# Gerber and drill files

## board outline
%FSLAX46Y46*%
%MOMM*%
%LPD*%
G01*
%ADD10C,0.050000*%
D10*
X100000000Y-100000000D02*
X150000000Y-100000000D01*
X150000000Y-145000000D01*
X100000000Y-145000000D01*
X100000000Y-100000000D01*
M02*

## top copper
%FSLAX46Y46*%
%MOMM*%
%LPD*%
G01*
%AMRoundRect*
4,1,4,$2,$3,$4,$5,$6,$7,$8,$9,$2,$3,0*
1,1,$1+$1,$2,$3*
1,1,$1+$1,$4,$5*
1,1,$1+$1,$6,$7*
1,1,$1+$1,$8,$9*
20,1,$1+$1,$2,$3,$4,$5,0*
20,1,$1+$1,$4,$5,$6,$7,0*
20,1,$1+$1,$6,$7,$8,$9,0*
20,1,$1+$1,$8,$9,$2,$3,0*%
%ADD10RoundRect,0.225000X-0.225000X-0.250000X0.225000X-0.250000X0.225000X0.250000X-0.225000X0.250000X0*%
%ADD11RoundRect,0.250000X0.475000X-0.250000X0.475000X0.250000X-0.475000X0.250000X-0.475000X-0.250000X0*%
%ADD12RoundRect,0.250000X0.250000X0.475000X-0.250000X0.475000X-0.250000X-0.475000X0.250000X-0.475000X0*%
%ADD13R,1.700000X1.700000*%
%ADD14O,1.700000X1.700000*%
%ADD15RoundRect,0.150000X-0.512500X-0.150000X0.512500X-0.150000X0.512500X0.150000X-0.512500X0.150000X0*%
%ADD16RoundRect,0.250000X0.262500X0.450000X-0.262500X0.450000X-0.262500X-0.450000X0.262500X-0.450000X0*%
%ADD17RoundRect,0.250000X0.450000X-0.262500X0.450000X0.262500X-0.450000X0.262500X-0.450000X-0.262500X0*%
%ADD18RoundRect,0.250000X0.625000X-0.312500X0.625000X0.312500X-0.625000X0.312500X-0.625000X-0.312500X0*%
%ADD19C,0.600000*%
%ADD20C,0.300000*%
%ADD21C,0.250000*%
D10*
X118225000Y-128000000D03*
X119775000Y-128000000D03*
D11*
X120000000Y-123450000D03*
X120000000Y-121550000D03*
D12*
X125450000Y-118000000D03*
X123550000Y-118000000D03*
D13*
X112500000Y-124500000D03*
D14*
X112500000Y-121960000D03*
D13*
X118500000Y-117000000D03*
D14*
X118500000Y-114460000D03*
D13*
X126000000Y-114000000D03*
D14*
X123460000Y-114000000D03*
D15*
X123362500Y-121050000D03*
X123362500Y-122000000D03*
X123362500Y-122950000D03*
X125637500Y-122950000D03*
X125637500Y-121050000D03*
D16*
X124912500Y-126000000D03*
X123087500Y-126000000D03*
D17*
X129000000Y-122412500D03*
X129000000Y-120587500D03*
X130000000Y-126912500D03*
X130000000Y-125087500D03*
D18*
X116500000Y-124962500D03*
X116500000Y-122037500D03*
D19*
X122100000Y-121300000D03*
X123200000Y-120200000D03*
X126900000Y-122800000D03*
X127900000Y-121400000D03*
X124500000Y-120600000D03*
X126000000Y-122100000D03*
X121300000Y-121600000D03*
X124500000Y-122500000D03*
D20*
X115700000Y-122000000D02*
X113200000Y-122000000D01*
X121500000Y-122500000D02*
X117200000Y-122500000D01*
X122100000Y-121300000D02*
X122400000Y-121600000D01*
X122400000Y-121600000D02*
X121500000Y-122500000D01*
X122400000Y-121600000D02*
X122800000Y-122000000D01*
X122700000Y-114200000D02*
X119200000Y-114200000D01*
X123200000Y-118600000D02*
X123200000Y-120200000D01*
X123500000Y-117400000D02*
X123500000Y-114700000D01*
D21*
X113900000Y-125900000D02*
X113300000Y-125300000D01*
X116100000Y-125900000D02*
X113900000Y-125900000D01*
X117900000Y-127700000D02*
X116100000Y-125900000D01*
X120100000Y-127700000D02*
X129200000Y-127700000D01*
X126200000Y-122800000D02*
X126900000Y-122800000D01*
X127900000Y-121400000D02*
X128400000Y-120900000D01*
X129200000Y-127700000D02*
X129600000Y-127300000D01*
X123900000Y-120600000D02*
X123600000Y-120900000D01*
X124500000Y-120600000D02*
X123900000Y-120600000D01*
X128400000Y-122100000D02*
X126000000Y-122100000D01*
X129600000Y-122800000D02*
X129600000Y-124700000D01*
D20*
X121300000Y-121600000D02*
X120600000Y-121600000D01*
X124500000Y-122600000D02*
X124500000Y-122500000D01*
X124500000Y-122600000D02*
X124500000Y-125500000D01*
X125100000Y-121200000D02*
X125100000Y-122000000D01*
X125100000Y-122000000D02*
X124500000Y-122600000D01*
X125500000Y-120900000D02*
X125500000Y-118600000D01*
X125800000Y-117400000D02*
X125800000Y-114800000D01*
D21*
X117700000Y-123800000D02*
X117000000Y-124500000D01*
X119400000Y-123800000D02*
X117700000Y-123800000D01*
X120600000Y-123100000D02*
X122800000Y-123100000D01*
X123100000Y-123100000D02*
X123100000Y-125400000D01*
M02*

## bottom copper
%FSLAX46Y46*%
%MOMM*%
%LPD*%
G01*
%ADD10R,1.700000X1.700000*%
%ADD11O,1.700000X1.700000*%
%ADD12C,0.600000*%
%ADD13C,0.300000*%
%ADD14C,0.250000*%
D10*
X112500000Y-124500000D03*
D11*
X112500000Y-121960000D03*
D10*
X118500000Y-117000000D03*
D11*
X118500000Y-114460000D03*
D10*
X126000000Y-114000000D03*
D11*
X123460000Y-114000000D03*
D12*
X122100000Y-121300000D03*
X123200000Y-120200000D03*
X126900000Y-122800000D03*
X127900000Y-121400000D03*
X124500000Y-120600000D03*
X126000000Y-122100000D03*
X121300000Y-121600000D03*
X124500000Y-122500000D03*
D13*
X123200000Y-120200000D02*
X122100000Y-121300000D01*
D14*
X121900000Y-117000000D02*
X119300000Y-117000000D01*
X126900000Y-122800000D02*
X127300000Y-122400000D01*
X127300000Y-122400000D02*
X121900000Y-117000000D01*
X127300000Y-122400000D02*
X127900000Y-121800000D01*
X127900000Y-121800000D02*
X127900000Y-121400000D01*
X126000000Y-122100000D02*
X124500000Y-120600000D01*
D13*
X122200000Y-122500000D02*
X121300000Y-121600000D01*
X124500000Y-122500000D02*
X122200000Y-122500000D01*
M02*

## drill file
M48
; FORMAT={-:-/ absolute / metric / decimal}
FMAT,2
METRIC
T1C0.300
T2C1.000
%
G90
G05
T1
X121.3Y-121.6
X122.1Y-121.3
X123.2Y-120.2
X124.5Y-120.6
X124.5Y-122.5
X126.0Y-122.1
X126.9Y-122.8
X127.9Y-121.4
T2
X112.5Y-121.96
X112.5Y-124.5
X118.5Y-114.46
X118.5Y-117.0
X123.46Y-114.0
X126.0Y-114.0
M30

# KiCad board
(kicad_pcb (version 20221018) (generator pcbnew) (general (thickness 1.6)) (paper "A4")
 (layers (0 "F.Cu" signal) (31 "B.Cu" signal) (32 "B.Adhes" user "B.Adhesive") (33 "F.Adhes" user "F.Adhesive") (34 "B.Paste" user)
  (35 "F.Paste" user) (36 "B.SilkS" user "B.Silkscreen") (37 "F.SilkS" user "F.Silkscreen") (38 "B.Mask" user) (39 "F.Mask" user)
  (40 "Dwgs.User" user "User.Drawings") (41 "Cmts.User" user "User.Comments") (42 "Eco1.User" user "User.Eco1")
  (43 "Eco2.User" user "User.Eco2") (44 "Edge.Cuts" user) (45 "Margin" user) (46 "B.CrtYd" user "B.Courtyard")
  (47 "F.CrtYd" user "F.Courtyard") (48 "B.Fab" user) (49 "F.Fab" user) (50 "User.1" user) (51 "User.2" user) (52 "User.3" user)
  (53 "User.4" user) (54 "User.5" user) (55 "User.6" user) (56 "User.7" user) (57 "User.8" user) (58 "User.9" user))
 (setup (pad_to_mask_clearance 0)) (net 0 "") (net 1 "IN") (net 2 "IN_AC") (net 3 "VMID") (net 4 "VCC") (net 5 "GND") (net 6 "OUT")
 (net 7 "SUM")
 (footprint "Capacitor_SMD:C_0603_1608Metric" (layer "F.Cu") (at 119 128)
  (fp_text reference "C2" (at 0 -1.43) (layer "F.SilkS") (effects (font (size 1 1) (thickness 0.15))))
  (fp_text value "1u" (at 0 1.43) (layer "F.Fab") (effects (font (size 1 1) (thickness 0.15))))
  (pad "1" smd roundrect (at -0.775 0) (size 0.9 0.95) (layers "F.Cu" "F.Paste" "F.Mask") (roundrect_rratio 0.25) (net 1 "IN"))
  (pad "2" smd roundrect (at 0.775 0) (size 0.9 0.95) (layers "F.Cu" "F.Paste" "F.Mask") (roundrect_rratio 0.25) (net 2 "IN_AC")))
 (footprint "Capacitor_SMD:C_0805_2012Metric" (layer "F.Cu") (at 120 122.5 90)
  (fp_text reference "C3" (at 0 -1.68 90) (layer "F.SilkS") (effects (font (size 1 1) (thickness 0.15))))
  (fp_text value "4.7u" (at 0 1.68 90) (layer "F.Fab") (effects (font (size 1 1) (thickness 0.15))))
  (pad "1" smd roundrect (at -0.95 0 90) (size 1 1.45) (layers "F.Cu" "F.Paste" "F.Mask") (roundrect_rratio 0.25) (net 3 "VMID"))
  (pad "2" smd roundrect (at 0.95 0 90) (size 1 1.45) (layers "F.Cu" "F.Paste" "F.Mask") (roundrect_rratio 0.25) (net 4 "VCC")))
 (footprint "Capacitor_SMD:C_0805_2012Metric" (layer "F.Cu") (at 124.5 118 180)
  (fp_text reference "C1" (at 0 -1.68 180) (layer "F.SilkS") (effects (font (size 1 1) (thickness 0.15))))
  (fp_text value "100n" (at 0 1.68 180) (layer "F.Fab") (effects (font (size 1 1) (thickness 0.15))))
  (pad "1" smd roundrect (at -0.95 0 180) (size 1 1.45) (layers "F.Cu" "F.Paste" "F.Mask") (roundrect_rratio 0.25) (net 4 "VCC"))
  (pad "2" smd roundrect (at 0.95 0 180) (size 1 1.45) (layers "F.Cu" "F.Paste" "F.Mask") (roundrect_rratio 0.25) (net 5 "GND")))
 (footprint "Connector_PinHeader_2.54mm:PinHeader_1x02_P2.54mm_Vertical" (layer "F.Cu") (at 112.5 124.5 180)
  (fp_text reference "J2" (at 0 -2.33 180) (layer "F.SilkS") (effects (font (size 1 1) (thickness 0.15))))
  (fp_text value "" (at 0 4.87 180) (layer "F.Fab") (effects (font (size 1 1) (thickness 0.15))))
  (pad "1" thru_hole rect (at 0 0 180) (size 1.7 1.7) (drill 1) (layers "*.Cu" "*.Mask") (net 1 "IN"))
  (pad "2" thru_hole oval (at 0 2.54 180) (size 1.7 1.7) (drill 1) (layers "*.Cu" "*.Mask") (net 5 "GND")))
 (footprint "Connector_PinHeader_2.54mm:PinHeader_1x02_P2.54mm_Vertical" (layer "F.Cu") (at 118.5 117 180)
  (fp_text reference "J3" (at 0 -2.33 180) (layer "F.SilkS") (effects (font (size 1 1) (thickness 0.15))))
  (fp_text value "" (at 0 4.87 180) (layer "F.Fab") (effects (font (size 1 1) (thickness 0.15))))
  (pad "1" thru_hole rect (at 0 0 180) (size 1.7 1.7) (drill 1) (layers "*.Cu" "*.Mask") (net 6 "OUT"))
  (pad "2" thru_hole oval (at 0 2.54 180) (size 1.7 1.7) (drill 1) (layers "*.Cu" "*.Mask") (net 5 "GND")))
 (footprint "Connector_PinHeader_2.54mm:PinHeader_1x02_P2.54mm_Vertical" (layer "F.Cu") (at 126 114 -90)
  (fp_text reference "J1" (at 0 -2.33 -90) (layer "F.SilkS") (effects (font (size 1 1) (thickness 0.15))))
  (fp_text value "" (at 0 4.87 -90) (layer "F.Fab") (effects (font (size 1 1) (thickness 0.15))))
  (pad "1" thru_hole rect (at 0 0 270) (size 1.7 1.7) (drill 1) (layers "*.Cu" "*.Mask") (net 4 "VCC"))
  (pad "2" thru_hole oval (at 0 2.54 270) (size 1.7 1.7) (drill 1) (layers "*.Cu" "*.Mask") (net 5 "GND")))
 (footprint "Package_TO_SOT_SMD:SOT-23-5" (layer "F.Cu") (at 124.5 122)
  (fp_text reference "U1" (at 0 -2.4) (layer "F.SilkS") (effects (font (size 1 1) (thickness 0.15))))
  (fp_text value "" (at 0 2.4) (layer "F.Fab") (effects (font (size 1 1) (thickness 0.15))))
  (pad "1" smd roundrect (at -1.1375 -0.95) (size 1.325 0.6) (layers "F.Cu" "F.Paste" "F.Mask") (roundrect_rratio 0.25) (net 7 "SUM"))
  (pad "2" smd roundrect (at -1.1375 0) (size 1.325 0.6) (layers "F.Cu" "F.Paste" "F.Mask") (roundrect_rratio 0.25) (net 5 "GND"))
  (pad "3" smd roundrect (at -1.1375 0.95) (size 1.325 0.6) (layers "F.Cu" "F.Paste" "F.Mask") (roundrect_rratio 0.25) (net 3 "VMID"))
  (pad "4" smd roundrect (at 1.1375 0.95) (size 1.325 0.6) (layers "F.Cu" "F.Paste" "F.Mask") (roundrect_rratio 0.25) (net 6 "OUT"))
  (pad "5" smd roundrect (at 1.1375 -0.95) (size 1.325 0.6) (layers "F.Cu" "F.Paste" "F.Mask") (roundrect_rratio 0.25) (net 4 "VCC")))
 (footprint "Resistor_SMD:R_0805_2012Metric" (layer "F.Cu") (at 124 126 180)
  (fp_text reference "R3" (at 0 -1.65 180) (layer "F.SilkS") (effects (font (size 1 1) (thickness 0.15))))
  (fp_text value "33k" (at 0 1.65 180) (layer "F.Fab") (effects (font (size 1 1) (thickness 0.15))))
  (pad "1" smd roundrect (at -0.9125 0 180) (size 1.025 1.4) (layers "F.Cu" "F.Paste" "F.Mask") (roundrect_rratio 0.243902) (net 4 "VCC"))
  (pad "2" smd roundrect (at 0.9125 0 180) (size 1.025 1.4) (layers "F.Cu" "F.Paste" "F.Mask") (roundrect_rratio 0.243902) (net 3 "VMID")))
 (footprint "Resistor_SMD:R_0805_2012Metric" (layer "F.Cu") (at 129 121.5 90)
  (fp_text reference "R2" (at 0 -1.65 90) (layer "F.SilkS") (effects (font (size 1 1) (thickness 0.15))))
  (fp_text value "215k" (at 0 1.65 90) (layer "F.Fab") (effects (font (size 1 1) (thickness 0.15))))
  (pad "1" smd roundrect (at -0.9125 0 90) (size 1.025 1.4) (layers "F.Cu" "F.Paste" "F.Mask") (roundrect_rratio 0.243902) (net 7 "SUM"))
  (pad "2" smd roundrect (at 0.9125 0 90) (size 1.025 1.4) (layers "F.Cu" "F.Paste" "F.Mask") (roundrect_rratio 0.243902) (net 6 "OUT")))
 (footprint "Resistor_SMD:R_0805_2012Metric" (layer "F.Cu") (at 130 126 90)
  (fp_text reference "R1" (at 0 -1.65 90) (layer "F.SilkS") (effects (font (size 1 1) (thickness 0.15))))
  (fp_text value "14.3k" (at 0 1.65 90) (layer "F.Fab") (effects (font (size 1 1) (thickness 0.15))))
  (pad "1" smd roundrect (at -0.9125 0 90) (size 1.025 1.4) (layers "F.Cu" "F.Paste" "F.Mask") (roundrect_rratio 0.243902) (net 2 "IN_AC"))
  (pad "2" smd roundrect (at 0.9125 0 90) (size 1.025 1.4) (layers "F.Cu" "F.Paste" "F.Mask") (roundrect_rratio 0.243902) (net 7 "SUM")))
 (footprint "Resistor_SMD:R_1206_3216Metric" (layer "F.Cu") (at 116.5 123.5 90)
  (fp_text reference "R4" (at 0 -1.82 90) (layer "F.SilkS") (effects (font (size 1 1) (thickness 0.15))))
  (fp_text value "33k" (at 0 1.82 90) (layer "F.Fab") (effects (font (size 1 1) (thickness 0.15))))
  (pad "1" smd roundrect (at -1.4625 0 90) (size 1.125 1.75) (layers "F.Cu" "F.Paste" "F.Mask") (roundrect_rratio 0.222222) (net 3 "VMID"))
  (pad "2" smd roundrect (at 1.4625 0 90) (size 1.125 1.75) (layers "F.Cu" "F.Paste" "F.Mask") (roundrect_rratio 0.222222) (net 5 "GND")))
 (gr_rect (start 100 100) (end 150 145) (stroke (width 0.05) (type default)) (fill none) (layer "Edge.Cuts"))
 (segment (start 115.7 122) (end 113.2 122) (width 0.3) (layer "F.Cu") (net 5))
 (segment (start 121.5 122.5) (end 117.2 122.5) (width 0.3) (layer "F.Cu") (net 5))
 (segment (start 122.1 121.3) (end 122.4 121.6) (width 0.3) (layer "F.Cu") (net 5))
 (segment (start 122.4 121.6) (end 121.5 122.5) (width 0.3) (layer "F.Cu") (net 5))
 (segment (start 122.4 121.6) (end 122.8 122) (width 0.3) (layer "F.Cu") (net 5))
 (segment (start 122.7 114.2) (end 119.2 114.2) (width 0.3) (layer "F.Cu") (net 5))
 (segment (start 123.2 118.6) (end 123.2 120.2) (width 0.3) (layer "F.Cu") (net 5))
 (segment (start 123.5 117.4) (end 123.5 114.7) (width 0.3) (layer "F.Cu") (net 5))
 (via (at 122.1 121.3) (size 0.6) (drill 0.3) (layers "F.Cu" "B.Cu") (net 5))
 (via (at 123.2 120.2) (size 0.6) (drill 0.3) (layers "F.Cu" "B.Cu") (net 5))
 (segment (start 113.9 125.9) (end 113.3 125.3) (width 0.25) (layer "F.Cu") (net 1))
 (segment (start 116.1 125.9) (end 113.9 125.9) (width 0.25) (layer "F.Cu") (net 1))
 (segment (start 117.9 127.7) (end 116.1 125.9) (width 0.25) (layer "F.Cu") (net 1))
 (segment (start 120.1 127.7) (end 129.2 127.7) (width 0.25) (layer "F.Cu") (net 2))
 (segment (start 123.2 120.2) (end 122.1 121.3) (width 0.3) (layer "B.Cu") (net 5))
 (segment (start 126.2 122.8) (end 126.9 122.8) (width 0.25) (layer "F.Cu") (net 6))
 (segment (start 127.9 121.4) (end 128.4 120.9) (width 0.25) (layer "F.Cu") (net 6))
 (segment (start 129.2 127.7) (end 129.6 127.3) (width 0.25) (layer "F.Cu") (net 2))
 (via (at 126.9 122.8) (size 0.6) (drill 0.3) (layers "F.Cu" "B.Cu") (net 6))
 (via (at 127.9 121.4) (size 0.6) (drill 0.3) (layers "F.Cu" "B.Cu") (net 6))
 (segment (start 121.9 117) (end 119.3 117) (width 0.25) (layer "B.Cu") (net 6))
 (segment (start 123.9 120.6) (end 123.6 120.9) (width 0.25) (layer "F.Cu") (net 7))
 (segment (start 124.5 120.6) (end 123.9 120.6) (width 0.25) (layer "F.Cu") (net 7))
 (segment (start 126.9 122.8) (end 127.3 122.4) (width 0.25) (layer "B.Cu") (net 6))
 (segment (start 127.3 122.4) (end 121.9 117) (width 0.25) (layer "B.Cu") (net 6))
 (segment (start 127.3 122.4) (end 127.9 121.8) (width 0.25) (layer "B.Cu") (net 6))
 (segment (start 127.9 121.8) (end 127.9 121.4) (width 0.25) (layer "B.Cu") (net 6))
 (segment (start 128.4 122.1) (end 126 122.1) (width 0.25) (layer "F.Cu") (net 7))
 (segment (start 129.6 122.8) (end 129.6 124.7) (width 0.25) (layer "F.Cu") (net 7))
 (via (at 124.5 120.6) (size 0.6) (drill 0.3) (layers "F.Cu" "B.Cu") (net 7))
 (via (at 126 122.1) (size 0.6) (drill 0.3) (layers "F.Cu" "B.Cu") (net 7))
 (segment (start 121.3 121.6) (end 120.6 121.6) (width 0.3) (layer "F.Cu") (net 4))
 (segment (start 124.5 122.6) (end 124.5 122.5) (width 0.3) (layer "F.Cu") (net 4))
 (segment (start 124.5 122.6) (end 124.5 125.5) (width 0.3) (layer "F.Cu") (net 4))
 (segment (start 125.1 121.2) (end 125.1 122) (width 0.3) (layer "F.Cu") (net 4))
 (segment (start 125.1 122) (end 124.5 122.6) (width 0.3) (layer "F.Cu") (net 4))
 (segment (start 125.5 120.9) (end 125.5 118.6) (width 0.3) (layer "F.Cu") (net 4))
 (segment (start 125.8 117.4) (end 125.8 114.8) (width 0.3) (layer "F.Cu") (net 4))
 (segment (start 126 122.1) (end 124.5 120.6) (width 0.25) (layer "B.Cu") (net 7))
 (via (at 121.3 121.6) (size 0.6) (drill 0.3) (layers "F.Cu" "B.Cu") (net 4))
 (via (at 124.5 122.5) (size 0.6) (drill 0.3) (layers "F.Cu" "B.Cu") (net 4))
 (segment (start 117.7 123.8) (end 117 124.5) (width 0.25) (layer "F.Cu") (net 3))
 (segment (start 119.4 123.8) (end 117.7 123.8) (width 0.25) (layer "F.Cu") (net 3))
 (segment (start 120.6 123.1) (end 122.8 123.1) (width 0.25) (layer "F.Cu") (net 3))
 (segment (start 122.2 122.5) (end 121.3 121.6) (width 0.3) (layer "B.Cu") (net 4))
 (segment (start 123.1 123.1) (end 123.1 125.4) (width 0.25) (layer "F.Cu") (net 3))
 (segment (start 124.5 122.5) (end 122.2 122.5) (width 0.3) (layer "B.Cu") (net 4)))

